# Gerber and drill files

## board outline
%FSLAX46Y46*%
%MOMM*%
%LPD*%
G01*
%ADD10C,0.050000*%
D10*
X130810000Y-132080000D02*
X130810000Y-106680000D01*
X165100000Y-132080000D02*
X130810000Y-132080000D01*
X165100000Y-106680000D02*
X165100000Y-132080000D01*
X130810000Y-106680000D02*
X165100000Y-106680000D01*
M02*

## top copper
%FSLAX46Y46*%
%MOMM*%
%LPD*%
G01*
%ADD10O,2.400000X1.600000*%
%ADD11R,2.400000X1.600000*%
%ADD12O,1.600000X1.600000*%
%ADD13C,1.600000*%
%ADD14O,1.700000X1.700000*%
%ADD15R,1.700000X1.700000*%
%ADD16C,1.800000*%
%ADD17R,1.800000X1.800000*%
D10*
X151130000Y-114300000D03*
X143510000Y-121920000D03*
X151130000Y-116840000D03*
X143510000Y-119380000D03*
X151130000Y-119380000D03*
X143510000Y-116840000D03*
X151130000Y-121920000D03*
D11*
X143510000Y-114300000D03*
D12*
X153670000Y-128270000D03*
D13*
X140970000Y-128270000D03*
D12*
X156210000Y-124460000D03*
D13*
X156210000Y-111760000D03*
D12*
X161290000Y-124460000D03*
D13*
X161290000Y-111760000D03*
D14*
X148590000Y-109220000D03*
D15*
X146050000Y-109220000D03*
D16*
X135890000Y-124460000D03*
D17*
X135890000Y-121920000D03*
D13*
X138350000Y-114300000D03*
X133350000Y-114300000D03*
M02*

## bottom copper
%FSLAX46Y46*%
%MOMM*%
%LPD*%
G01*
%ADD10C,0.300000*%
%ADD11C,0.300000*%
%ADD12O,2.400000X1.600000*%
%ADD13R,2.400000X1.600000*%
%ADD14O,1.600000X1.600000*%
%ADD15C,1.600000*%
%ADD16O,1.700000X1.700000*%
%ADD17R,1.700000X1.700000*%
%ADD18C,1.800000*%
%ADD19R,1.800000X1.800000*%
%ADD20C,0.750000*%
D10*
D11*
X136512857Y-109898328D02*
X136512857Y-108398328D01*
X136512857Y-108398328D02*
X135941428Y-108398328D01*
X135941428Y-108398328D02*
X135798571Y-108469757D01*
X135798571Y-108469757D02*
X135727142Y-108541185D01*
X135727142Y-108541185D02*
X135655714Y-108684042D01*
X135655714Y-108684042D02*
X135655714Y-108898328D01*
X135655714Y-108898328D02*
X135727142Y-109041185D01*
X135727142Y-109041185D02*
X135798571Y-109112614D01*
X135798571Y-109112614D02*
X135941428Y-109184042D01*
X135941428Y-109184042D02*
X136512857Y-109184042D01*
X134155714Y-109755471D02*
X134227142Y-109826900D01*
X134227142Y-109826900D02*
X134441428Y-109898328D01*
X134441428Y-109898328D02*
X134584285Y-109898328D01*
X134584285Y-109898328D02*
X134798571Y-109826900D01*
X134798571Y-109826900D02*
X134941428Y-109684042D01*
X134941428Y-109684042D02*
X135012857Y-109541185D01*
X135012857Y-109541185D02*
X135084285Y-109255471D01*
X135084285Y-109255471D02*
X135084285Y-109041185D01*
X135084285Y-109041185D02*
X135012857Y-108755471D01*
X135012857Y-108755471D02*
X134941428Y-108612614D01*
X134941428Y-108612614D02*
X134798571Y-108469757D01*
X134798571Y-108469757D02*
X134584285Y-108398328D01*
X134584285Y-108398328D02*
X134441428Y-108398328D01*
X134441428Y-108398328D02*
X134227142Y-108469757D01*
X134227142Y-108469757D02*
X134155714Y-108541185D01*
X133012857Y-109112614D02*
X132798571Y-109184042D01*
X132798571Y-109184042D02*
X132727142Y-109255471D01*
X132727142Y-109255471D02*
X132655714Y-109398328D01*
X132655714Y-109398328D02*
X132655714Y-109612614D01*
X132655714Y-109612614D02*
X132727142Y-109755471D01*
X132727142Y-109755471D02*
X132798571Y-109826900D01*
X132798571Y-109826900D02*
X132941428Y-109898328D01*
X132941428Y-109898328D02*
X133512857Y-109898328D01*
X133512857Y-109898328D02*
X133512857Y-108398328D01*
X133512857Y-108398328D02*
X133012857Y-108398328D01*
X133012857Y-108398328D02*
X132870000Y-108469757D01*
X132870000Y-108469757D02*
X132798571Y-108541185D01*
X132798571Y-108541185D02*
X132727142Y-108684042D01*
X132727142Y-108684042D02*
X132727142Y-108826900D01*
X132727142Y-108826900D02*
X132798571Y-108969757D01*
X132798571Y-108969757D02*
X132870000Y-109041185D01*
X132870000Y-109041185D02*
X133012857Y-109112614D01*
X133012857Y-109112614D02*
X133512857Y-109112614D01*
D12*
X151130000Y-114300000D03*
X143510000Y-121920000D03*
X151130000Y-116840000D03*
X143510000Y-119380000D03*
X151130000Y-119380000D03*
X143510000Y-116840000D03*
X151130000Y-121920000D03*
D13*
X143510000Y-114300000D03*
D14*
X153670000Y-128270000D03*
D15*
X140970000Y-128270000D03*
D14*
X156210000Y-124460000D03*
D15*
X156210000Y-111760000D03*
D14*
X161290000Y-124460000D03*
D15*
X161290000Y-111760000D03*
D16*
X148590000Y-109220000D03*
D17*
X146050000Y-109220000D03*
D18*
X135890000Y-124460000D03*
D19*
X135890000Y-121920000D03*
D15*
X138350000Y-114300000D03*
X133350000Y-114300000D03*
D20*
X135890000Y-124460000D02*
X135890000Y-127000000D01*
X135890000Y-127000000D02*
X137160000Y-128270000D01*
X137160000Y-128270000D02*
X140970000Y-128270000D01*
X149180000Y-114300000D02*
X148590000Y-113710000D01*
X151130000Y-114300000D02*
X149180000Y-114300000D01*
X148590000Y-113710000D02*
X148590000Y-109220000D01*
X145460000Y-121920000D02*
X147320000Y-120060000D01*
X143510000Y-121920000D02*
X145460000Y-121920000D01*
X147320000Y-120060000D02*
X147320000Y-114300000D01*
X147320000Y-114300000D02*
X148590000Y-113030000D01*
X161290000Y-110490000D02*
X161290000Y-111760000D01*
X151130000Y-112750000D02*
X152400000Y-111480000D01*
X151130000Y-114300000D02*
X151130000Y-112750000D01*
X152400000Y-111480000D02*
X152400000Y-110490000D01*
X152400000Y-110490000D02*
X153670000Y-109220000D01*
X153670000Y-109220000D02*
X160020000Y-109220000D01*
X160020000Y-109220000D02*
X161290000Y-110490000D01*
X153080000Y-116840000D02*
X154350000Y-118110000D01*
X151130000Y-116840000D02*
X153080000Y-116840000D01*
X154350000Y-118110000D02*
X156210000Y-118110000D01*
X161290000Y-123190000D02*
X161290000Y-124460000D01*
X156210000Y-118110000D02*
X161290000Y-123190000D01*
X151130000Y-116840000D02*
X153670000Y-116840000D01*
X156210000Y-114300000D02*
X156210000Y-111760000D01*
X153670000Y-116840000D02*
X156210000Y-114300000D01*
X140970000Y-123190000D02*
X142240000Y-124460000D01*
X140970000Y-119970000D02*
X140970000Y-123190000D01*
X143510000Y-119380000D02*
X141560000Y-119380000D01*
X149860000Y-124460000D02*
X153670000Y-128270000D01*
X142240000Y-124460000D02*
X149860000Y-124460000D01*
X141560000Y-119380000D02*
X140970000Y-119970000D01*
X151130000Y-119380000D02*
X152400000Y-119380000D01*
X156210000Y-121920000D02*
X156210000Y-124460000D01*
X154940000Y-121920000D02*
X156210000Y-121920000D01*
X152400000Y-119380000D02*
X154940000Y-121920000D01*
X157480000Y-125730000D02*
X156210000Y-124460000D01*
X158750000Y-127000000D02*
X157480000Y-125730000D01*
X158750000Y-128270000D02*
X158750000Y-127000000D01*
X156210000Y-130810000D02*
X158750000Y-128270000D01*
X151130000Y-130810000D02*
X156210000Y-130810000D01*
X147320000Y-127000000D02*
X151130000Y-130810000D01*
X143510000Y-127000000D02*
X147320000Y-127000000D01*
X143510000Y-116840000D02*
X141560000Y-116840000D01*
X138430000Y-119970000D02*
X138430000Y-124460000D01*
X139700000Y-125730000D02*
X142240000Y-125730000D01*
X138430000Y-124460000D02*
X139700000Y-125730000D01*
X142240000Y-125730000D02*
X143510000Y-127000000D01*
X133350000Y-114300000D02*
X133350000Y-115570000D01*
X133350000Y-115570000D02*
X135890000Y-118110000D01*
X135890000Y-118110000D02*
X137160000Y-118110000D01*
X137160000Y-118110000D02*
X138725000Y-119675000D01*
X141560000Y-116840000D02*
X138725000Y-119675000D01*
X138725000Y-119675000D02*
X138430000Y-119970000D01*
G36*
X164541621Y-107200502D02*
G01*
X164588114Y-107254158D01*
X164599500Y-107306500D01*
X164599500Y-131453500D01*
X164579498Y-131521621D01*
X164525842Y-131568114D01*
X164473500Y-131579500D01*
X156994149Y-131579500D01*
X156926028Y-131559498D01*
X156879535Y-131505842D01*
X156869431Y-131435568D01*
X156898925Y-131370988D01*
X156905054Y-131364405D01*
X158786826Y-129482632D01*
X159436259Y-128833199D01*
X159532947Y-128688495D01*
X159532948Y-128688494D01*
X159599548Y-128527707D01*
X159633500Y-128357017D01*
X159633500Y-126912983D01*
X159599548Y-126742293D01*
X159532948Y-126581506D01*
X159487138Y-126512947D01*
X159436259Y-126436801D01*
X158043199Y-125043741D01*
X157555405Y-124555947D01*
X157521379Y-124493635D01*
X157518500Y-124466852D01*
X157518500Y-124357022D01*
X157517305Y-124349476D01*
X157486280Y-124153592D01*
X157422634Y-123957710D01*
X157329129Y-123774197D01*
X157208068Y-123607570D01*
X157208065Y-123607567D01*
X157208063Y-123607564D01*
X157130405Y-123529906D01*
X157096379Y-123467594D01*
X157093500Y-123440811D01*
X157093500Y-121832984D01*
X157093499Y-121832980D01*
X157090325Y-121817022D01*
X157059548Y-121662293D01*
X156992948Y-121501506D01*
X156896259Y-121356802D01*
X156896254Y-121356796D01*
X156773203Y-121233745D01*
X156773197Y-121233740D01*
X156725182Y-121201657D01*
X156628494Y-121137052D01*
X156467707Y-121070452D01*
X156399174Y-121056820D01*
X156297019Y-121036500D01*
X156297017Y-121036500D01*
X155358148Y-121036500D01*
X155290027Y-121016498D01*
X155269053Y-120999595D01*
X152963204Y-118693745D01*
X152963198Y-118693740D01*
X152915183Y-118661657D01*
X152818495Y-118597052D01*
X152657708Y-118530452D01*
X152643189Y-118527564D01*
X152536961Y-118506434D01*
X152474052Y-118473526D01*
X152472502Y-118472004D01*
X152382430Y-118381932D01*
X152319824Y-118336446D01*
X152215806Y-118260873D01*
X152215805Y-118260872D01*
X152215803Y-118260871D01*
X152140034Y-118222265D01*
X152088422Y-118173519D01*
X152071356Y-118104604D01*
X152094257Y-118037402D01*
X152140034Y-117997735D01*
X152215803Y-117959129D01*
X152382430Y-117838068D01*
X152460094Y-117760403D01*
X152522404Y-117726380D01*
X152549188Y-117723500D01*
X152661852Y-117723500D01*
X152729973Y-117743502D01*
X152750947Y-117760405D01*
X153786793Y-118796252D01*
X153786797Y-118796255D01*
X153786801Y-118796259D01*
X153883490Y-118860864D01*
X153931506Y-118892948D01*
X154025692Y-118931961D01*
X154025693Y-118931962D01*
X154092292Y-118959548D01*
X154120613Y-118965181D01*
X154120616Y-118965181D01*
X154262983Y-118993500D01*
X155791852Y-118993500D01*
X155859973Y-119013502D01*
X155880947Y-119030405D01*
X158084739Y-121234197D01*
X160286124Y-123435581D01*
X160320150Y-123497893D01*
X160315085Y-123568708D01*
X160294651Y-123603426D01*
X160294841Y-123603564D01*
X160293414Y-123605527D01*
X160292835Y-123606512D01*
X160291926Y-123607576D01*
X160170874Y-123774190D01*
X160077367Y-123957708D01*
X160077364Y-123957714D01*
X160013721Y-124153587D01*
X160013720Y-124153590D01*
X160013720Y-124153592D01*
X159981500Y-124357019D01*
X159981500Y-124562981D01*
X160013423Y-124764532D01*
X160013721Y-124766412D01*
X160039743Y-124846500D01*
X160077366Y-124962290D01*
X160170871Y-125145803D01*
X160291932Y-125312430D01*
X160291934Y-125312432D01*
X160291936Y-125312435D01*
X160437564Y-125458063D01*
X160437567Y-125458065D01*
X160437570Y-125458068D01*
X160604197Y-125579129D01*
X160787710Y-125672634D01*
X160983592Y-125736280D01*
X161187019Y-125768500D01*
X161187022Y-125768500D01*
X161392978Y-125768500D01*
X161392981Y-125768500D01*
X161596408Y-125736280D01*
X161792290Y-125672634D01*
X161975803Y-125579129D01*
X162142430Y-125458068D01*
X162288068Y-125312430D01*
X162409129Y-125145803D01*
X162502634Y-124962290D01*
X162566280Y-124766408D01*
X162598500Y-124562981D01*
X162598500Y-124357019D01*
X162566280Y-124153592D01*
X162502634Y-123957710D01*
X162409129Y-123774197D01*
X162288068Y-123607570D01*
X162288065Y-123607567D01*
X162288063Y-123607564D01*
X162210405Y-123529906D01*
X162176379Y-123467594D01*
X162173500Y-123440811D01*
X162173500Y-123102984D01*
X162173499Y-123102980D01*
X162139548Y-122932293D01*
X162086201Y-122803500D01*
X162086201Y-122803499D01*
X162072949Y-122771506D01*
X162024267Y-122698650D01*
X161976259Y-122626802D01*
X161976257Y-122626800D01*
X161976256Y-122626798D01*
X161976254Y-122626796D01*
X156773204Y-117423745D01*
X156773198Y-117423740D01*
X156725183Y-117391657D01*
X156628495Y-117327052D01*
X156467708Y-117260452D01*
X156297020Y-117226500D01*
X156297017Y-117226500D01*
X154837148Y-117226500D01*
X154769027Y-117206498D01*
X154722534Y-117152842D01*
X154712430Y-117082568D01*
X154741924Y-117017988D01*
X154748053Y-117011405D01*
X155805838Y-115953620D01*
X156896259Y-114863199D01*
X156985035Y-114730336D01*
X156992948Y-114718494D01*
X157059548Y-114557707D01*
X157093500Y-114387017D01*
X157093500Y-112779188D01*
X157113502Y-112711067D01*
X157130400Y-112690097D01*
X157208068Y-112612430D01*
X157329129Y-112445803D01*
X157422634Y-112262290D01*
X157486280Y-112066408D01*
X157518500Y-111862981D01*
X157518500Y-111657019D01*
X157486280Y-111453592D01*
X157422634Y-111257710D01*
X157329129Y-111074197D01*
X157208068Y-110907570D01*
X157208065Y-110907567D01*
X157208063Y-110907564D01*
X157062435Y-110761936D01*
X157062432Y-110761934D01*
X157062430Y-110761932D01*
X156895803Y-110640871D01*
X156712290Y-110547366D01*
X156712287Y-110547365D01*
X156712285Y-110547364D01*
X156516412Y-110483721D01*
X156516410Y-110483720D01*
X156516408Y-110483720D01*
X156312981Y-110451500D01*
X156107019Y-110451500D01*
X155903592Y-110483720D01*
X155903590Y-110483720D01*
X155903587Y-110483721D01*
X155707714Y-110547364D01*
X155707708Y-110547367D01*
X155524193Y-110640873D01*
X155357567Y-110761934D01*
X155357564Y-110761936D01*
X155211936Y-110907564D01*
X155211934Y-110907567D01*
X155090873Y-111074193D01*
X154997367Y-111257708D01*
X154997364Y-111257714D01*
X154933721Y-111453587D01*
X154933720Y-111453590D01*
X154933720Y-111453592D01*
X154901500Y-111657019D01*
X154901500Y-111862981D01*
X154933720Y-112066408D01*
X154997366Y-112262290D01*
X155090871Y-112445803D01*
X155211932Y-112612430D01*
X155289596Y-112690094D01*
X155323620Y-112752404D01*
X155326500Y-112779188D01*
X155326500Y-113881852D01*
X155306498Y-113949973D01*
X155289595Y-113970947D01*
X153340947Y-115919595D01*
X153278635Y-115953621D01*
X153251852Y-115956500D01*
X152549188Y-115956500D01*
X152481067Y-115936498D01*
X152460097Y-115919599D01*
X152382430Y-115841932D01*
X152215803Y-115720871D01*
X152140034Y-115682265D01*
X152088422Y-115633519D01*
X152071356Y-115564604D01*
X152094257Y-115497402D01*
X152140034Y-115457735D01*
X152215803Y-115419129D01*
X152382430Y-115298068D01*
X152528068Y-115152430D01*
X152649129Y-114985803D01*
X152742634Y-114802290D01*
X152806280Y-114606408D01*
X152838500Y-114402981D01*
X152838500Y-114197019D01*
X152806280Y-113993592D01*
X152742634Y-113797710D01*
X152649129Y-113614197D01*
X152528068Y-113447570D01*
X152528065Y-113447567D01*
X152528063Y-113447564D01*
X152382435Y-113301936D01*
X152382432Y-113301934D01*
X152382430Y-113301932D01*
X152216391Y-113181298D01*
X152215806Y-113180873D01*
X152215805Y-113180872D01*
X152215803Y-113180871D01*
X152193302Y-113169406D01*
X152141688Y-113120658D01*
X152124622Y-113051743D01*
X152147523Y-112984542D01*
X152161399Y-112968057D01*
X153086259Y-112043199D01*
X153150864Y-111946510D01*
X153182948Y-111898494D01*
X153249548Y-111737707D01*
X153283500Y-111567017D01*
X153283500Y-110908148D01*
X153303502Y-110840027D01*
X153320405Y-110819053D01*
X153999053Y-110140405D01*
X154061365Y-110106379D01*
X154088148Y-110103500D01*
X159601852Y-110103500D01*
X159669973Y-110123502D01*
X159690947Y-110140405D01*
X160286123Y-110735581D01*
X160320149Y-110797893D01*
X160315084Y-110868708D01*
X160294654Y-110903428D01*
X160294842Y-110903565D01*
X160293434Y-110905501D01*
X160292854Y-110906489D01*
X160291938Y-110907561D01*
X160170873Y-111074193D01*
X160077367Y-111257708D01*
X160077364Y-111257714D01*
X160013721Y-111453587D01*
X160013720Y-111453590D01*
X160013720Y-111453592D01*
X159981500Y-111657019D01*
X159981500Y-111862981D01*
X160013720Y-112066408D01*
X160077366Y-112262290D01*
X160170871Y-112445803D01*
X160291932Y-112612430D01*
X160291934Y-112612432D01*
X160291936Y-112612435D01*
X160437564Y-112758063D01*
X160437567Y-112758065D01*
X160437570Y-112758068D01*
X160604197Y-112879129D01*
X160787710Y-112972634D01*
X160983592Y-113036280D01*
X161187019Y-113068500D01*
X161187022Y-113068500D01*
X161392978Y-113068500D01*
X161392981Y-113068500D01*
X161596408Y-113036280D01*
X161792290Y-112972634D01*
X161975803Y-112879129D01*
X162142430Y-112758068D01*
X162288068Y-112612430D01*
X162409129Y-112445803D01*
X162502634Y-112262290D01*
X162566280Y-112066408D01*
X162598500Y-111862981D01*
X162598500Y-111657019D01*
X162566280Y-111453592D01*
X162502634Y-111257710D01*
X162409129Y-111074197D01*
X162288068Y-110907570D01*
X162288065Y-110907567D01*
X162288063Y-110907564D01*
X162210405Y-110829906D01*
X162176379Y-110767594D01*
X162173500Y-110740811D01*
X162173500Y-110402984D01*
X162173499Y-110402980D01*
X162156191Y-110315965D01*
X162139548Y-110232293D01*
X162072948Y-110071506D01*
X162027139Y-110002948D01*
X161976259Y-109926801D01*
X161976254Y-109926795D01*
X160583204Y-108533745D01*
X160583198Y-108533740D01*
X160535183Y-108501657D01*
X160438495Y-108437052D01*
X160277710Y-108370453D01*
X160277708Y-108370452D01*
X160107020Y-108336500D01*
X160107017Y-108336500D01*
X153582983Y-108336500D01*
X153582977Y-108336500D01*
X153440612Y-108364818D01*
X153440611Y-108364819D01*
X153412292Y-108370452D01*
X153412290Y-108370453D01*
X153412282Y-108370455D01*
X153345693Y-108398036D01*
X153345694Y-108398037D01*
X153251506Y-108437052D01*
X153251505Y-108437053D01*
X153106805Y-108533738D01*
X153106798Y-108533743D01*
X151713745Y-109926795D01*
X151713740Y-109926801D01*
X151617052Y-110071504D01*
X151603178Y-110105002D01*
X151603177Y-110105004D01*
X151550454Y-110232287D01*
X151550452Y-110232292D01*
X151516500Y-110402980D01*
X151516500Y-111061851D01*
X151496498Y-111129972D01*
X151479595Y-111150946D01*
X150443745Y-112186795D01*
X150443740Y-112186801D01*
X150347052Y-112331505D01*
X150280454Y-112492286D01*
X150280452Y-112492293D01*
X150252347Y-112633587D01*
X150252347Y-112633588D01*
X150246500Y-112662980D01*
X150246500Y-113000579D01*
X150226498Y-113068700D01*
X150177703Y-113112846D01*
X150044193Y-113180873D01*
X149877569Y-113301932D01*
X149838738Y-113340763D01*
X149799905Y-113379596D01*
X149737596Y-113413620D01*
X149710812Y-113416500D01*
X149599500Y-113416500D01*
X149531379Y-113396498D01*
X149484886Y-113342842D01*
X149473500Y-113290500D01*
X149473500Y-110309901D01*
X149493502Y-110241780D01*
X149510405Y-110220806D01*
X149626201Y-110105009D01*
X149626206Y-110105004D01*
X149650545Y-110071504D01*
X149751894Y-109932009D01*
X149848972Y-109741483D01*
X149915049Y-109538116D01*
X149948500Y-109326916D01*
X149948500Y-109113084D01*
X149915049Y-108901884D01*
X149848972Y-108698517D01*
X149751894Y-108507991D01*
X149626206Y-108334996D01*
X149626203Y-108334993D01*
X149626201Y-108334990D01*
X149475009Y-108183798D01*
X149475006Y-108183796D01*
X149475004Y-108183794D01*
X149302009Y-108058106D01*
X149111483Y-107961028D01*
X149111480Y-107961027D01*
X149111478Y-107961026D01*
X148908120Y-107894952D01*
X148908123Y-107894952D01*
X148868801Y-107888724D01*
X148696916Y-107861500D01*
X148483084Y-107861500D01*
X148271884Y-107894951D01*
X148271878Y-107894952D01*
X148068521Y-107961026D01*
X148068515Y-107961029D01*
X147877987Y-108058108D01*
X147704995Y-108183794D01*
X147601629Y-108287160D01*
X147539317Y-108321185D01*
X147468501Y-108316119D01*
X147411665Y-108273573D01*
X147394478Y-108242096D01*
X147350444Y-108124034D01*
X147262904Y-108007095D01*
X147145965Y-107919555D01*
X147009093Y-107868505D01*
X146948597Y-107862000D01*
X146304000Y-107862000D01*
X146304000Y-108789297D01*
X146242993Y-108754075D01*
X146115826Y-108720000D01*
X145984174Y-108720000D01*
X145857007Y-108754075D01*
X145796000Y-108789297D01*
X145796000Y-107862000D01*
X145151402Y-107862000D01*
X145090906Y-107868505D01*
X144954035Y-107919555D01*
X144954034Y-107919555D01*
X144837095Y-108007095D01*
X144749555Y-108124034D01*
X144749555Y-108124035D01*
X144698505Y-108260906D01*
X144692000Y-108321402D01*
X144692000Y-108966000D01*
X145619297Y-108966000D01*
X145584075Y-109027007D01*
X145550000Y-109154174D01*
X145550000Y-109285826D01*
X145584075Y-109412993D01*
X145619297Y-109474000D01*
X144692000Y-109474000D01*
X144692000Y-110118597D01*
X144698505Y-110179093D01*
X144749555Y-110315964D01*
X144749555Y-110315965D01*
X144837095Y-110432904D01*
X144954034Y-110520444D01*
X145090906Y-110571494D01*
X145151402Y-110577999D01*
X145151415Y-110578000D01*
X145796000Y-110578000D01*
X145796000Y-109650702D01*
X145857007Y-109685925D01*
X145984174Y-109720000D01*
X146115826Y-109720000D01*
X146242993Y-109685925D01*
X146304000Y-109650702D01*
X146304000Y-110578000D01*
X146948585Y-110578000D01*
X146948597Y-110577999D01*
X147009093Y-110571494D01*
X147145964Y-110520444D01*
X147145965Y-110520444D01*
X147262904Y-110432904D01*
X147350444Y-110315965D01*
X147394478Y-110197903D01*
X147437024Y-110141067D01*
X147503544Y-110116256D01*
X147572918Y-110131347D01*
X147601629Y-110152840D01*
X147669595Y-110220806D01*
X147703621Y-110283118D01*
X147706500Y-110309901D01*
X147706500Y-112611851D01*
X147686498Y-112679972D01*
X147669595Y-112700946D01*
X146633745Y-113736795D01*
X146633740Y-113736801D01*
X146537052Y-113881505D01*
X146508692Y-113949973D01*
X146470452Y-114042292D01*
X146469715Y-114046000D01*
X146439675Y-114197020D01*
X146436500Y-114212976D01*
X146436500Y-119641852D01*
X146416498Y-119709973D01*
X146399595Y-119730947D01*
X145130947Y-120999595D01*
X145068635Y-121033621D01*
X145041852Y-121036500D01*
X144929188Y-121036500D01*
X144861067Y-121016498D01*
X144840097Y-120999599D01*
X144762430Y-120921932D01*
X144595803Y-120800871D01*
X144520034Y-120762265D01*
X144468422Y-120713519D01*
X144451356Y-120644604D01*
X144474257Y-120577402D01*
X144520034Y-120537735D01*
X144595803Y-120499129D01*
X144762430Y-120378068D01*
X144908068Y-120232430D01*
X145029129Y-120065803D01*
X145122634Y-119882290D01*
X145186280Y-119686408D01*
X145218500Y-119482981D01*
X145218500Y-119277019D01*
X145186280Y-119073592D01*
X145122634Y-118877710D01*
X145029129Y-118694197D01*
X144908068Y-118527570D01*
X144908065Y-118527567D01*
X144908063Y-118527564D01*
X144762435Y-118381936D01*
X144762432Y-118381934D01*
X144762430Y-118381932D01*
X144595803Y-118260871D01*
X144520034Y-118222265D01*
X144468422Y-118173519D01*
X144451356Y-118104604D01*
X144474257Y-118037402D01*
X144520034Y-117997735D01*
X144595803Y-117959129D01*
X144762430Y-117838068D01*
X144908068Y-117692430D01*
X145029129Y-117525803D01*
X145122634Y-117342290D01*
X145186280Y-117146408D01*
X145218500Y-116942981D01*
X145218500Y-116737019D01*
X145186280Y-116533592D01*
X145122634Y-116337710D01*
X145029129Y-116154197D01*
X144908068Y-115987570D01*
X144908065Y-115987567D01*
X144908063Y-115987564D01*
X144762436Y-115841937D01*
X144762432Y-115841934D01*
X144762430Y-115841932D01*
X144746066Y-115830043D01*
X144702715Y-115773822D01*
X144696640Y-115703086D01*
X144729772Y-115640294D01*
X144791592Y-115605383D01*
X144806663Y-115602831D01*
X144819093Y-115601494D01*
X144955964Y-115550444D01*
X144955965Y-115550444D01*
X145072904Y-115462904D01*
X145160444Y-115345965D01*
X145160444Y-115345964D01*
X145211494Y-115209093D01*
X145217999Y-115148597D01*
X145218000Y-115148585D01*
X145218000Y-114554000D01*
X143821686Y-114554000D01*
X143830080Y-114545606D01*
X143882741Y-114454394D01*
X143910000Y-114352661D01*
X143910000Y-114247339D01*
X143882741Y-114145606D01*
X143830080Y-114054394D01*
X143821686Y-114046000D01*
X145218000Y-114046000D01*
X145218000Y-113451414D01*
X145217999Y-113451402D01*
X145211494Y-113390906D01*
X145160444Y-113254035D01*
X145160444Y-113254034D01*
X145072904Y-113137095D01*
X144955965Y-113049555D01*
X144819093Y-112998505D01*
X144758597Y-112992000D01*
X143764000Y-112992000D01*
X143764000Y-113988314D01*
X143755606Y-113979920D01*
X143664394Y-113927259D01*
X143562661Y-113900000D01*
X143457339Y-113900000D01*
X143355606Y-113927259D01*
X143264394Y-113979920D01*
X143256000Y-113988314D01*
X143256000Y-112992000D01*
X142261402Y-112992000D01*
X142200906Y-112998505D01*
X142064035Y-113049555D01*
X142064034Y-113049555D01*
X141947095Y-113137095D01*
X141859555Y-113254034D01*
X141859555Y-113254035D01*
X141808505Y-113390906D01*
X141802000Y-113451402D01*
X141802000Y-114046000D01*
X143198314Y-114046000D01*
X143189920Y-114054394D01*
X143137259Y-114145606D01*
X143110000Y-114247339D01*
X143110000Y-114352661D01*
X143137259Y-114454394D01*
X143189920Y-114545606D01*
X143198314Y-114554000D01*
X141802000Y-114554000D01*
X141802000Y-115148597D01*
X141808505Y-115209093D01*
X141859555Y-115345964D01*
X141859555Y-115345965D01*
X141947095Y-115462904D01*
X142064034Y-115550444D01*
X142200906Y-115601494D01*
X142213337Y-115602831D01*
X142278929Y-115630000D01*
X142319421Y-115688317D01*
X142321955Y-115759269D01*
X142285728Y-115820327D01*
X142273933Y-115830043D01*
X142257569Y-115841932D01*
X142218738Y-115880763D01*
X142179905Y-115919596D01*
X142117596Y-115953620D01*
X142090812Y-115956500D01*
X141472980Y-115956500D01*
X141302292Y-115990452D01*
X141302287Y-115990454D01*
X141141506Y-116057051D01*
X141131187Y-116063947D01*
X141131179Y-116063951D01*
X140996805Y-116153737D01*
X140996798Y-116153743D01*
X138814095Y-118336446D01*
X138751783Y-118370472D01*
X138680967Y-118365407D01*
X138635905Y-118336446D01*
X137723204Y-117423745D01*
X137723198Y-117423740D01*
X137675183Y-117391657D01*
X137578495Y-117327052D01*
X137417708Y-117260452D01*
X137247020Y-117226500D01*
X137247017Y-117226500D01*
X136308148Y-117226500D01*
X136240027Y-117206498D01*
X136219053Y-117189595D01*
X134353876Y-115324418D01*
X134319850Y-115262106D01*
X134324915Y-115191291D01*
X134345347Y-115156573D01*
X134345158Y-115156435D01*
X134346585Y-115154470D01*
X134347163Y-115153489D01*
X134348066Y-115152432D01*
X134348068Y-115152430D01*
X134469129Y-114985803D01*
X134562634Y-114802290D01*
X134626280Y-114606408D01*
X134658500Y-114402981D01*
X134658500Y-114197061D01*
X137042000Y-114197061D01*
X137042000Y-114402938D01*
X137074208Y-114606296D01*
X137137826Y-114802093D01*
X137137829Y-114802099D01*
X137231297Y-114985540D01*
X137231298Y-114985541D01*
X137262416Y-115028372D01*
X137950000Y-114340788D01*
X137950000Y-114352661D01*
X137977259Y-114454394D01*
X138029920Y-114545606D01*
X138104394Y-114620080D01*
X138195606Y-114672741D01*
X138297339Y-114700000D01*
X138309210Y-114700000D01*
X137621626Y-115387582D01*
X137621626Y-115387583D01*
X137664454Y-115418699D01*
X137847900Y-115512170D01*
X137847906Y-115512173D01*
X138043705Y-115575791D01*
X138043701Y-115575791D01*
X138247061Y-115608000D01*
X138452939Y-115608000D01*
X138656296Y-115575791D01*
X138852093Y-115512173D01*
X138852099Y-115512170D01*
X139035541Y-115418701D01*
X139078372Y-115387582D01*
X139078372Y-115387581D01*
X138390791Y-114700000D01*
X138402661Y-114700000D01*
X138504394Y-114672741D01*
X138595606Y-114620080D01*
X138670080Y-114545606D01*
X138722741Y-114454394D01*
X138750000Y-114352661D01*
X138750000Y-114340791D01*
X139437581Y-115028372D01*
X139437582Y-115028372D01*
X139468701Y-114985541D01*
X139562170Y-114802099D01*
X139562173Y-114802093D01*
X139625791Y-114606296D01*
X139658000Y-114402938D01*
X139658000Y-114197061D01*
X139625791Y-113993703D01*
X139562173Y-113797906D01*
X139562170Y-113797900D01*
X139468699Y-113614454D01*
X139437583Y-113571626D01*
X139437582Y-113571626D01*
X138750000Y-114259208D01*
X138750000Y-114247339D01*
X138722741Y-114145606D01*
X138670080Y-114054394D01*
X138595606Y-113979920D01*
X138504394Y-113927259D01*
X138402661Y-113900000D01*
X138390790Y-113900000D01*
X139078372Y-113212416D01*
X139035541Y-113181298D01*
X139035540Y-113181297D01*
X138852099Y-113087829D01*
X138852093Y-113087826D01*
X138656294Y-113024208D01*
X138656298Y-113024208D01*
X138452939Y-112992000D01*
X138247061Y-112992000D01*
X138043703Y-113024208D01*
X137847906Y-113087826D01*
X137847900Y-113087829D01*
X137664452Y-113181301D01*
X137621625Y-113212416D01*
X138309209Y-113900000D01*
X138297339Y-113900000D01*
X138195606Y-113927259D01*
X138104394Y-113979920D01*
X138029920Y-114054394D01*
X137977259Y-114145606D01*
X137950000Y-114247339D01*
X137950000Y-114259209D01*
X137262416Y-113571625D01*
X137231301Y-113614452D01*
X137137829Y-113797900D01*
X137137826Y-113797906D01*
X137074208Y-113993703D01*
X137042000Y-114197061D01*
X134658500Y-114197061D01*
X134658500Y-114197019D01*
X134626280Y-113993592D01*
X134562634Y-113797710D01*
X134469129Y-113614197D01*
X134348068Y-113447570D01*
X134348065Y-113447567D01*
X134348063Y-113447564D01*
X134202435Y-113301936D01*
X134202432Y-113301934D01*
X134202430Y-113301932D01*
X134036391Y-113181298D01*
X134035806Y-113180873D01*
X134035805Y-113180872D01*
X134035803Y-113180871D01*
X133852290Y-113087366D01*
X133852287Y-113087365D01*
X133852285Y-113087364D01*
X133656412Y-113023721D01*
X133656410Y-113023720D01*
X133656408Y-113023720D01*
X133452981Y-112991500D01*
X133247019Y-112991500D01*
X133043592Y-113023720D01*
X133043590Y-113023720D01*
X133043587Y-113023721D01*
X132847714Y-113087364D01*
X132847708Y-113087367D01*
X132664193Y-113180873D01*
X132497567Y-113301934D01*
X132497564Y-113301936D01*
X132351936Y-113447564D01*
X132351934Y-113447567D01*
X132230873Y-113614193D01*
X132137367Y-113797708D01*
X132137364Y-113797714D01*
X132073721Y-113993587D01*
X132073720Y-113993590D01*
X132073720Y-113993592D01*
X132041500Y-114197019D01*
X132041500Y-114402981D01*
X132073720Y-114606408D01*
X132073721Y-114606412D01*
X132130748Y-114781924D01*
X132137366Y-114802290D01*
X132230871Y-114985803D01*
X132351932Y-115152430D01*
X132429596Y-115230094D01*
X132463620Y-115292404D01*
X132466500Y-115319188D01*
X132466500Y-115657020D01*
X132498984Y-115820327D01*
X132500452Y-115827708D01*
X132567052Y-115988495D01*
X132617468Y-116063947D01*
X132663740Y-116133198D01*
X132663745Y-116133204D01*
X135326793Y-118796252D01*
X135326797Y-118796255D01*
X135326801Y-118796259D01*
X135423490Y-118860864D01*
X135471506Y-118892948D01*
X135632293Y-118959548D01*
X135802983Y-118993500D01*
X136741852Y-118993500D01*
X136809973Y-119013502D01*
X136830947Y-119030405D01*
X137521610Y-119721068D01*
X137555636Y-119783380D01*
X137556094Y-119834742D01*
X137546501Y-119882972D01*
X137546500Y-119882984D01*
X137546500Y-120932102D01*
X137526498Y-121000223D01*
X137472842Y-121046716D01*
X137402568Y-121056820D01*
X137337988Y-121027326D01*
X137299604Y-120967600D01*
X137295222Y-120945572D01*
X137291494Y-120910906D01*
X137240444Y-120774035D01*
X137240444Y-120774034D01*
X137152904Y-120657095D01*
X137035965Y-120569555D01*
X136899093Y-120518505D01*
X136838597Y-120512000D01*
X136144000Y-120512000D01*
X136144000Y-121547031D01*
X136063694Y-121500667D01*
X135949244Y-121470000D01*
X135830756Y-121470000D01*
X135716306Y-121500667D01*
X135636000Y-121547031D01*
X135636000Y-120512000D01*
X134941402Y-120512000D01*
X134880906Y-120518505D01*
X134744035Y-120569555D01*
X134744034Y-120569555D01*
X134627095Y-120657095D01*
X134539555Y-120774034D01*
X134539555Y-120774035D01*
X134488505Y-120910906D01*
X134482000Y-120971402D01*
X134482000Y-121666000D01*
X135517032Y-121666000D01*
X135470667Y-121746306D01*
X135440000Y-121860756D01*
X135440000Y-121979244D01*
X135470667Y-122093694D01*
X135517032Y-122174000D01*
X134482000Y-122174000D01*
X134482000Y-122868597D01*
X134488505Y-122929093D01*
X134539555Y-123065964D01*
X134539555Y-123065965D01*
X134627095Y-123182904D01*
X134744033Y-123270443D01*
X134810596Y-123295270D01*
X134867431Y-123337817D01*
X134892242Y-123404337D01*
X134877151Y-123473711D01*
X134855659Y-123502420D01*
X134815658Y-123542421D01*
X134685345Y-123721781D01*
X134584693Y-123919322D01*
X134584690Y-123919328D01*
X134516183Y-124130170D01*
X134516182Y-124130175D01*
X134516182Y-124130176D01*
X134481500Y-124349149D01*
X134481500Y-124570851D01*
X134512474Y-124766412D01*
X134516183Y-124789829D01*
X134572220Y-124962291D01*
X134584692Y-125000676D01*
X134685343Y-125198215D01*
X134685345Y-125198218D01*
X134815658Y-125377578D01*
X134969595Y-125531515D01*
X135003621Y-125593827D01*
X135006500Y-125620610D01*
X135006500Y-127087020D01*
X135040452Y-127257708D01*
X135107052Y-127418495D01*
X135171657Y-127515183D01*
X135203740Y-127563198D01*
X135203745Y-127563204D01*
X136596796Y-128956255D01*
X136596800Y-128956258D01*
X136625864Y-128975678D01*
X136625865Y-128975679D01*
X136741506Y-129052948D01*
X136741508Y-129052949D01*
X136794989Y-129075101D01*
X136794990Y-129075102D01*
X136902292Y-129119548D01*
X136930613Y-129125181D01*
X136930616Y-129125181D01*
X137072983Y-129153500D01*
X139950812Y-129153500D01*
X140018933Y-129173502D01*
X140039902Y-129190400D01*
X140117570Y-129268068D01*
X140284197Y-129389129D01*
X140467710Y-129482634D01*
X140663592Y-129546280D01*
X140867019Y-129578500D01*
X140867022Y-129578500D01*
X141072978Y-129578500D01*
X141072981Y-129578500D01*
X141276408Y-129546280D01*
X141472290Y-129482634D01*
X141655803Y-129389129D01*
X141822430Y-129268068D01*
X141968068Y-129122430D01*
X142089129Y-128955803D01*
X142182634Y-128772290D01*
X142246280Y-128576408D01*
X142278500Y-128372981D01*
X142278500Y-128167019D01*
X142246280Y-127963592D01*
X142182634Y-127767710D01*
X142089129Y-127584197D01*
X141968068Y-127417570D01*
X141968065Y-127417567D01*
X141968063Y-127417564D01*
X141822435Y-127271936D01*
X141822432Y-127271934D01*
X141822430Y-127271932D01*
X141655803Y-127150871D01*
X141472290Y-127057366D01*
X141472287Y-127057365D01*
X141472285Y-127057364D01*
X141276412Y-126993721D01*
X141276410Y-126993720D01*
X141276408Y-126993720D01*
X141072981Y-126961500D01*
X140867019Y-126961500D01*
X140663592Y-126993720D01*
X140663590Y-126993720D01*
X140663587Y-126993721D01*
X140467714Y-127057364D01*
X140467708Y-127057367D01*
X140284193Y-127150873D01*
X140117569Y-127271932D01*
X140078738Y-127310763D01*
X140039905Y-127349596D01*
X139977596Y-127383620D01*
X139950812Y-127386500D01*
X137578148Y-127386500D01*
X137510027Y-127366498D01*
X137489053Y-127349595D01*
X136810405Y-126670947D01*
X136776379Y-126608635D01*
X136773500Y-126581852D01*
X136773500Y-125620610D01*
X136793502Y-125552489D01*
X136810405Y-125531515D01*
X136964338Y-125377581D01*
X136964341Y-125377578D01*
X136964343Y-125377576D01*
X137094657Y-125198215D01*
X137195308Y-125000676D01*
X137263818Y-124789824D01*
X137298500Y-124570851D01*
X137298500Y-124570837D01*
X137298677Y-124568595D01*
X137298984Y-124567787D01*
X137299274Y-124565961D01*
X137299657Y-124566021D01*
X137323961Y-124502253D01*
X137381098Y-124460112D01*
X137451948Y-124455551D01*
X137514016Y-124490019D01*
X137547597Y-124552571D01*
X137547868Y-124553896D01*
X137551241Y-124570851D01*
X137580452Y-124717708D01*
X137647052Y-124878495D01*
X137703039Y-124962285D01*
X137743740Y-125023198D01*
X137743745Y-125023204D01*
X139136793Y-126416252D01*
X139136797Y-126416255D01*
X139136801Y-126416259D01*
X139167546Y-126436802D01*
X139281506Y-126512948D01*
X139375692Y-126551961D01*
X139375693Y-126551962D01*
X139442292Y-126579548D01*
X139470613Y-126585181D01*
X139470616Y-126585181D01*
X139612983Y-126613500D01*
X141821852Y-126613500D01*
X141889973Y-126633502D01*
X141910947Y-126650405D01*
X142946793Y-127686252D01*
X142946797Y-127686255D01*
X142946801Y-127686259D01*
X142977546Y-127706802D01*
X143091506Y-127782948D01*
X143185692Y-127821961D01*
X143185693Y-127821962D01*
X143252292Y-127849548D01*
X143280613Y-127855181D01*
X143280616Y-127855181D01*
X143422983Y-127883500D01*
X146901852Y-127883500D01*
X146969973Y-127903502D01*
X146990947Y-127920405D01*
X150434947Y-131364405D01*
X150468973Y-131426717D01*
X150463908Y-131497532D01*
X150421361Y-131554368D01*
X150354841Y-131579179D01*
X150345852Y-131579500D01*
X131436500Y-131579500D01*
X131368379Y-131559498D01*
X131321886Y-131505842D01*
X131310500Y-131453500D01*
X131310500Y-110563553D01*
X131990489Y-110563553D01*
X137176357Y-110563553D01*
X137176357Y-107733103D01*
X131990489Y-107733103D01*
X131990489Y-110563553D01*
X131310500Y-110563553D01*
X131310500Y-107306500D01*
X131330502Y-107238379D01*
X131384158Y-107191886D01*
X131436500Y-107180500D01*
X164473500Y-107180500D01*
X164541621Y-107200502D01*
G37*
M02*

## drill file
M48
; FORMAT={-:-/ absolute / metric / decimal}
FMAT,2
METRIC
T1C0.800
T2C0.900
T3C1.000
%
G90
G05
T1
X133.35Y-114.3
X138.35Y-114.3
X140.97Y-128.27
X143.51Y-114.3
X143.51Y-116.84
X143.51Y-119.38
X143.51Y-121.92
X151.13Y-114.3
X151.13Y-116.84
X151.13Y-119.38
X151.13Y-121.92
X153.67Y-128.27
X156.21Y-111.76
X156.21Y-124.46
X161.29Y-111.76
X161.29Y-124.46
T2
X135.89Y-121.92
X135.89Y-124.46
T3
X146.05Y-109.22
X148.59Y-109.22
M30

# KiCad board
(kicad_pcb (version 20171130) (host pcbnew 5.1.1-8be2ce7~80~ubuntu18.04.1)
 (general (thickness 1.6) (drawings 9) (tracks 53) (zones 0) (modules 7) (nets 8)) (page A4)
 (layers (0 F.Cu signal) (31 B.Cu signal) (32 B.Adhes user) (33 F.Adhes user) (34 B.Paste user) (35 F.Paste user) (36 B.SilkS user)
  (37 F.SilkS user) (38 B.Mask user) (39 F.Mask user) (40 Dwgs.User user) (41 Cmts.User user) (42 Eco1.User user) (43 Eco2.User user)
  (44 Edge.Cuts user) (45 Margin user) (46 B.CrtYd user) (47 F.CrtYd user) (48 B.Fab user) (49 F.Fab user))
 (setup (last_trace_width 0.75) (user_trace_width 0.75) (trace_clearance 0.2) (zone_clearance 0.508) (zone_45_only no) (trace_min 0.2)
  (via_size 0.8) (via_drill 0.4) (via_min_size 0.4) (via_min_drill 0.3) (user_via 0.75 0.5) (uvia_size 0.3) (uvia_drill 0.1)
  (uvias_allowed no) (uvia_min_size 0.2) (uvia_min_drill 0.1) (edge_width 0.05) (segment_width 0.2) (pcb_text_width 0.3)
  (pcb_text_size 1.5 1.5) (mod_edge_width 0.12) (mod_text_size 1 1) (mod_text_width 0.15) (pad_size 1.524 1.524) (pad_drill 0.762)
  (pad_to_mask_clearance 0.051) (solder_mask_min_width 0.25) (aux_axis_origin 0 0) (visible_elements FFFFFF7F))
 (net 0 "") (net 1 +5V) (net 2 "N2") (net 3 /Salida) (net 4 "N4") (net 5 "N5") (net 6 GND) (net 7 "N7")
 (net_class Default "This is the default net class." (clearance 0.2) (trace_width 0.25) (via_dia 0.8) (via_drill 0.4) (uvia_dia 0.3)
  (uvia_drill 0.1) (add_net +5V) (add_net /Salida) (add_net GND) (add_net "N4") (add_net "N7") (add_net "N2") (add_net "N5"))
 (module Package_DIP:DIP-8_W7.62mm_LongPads (layer F.Cu) (at 143.51 114.3)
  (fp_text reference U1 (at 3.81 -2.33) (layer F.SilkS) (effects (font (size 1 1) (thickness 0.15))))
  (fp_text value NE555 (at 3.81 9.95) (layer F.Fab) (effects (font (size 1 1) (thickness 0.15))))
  (pad 8 thru_hole oval (at 7.62 0) (size 2.4 1.6) (drill 0.8) (layers *.Cu *.Mask) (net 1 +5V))
  (pad 4 thru_hole oval (at 0 7.62) (size 2.4 1.6) (drill 0.8) (layers *.Cu *.Mask) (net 1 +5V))
  (pad 7 thru_hole oval (at 7.62 2.54) (size 2.4 1.6) (drill 0.8) (layers *.Cu *.Mask) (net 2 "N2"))
  (pad 3 thru_hole oval (at 0 5.08) (size 2.4 1.6) (drill 0.8) (layers *.Cu *.Mask) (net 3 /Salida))
  (pad 6 thru_hole oval (at 7.62 5.08) (size 2.4 1.6) (drill 0.8) (layers *.Cu *.Mask) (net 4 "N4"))
  (pad 2 thru_hole oval (at 0 2.54) (size 2.4 1.6) (drill 0.8) (layers *.Cu *.Mask) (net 4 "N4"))
  (pad 5 thru_hole oval (at 7.62 7.62) (size 2.4 1.6) (drill 0.8) (layers *.Cu *.Mask) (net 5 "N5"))
  (pad 1 thru_hole rect (at 0 0) (size 2.4 1.6) (drill 0.8) (layers *.Cu *.Mask) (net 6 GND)))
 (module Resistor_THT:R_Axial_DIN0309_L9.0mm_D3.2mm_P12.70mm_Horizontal (layer F.Cu) (at 140.97 128.27)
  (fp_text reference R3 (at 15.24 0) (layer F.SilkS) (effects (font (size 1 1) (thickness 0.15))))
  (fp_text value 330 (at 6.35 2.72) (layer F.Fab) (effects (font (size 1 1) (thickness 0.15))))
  (pad 2 thru_hole oval (at 12.7 0) (size 1.6 1.6) (drill 0.8) (layers *.Cu *.Mask) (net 3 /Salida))
  (pad 1 thru_hole circle (at 0 0) (size 1.6 1.6) (drill 0.8) (layers *.Cu *.Mask) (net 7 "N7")))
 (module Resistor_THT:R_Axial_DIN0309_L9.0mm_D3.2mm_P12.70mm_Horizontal (layer F.Cu) (at 156.21 111.76 270)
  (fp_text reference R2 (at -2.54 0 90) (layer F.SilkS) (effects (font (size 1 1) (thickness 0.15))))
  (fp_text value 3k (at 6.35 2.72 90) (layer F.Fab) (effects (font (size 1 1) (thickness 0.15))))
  (pad 2 thru_hole oval (at 12.7 0 270) (size 1.6 1.6) (drill 0.8) (layers *.Cu *.Mask) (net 4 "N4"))
  (pad 1 thru_hole circle (at 0 0 270) (size 1.6 1.6) (drill 0.8) (layers *.Cu *.Mask) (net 2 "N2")))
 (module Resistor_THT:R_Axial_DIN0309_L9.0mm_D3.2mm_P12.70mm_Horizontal (layer F.Cu) (at 161.29 111.76 270)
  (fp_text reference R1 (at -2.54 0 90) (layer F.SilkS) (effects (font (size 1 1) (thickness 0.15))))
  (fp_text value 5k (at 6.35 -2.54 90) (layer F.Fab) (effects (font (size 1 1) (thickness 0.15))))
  (pad 2 thru_hole oval (at 12.7 0 270) (size 1.6 1.6) (drill 0.8) (layers *.Cu *.Mask) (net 2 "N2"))
  (pad 1 thru_hole circle (at 0 0 270) (size 1.6 1.6) (drill 0.8) (layers *.Cu *.Mask) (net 1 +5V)))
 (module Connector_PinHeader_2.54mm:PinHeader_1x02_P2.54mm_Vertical (layer F.Cu) (at 146.05 109.22 90)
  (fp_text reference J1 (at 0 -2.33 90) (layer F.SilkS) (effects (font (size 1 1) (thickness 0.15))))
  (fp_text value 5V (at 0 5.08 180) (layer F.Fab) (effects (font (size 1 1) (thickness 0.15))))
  (pad 2 thru_hole oval (at 0 2.54 90) (size 1.7 1.7) (drill 1) (layers *.Cu *.Mask) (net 1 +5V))
  (pad 1 thru_hole rect (at 0 0 90) (size 1.7 1.7) (drill 1) (layers *.Cu *.Mask) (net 6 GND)))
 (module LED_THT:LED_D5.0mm (layer F.Cu) (at 135.89 121.92 270)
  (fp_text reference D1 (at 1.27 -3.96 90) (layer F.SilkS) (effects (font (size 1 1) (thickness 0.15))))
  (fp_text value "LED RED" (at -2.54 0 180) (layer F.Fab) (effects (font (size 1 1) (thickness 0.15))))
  (pad 2 thru_hole circle (at 2.54 0 270) (size 1.8 1.8) (drill 0.9) (layers *.Cu *.Mask) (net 7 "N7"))
  (pad 1 thru_hole rect (at 0 0 270) (size 1.8 1.8) (drill 0.9) (layers *.Cu *.Mask) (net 6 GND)))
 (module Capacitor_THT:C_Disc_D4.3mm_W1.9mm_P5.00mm (layer F.Cu) (at 133.35 114.3)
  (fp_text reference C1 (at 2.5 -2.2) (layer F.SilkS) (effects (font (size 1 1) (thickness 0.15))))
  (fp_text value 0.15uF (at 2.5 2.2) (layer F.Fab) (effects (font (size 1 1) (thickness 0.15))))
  (pad 2 thru_hole circle (at 5 0) (size 1.6 1.6) (drill 0.8) (layers *.Cu *.Mask) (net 6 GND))
  (pad 1 thru_hole circle (at 0 0) (size 1.6 1.6) (drill 0.8) (layers *.Cu *.Mask) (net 4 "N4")))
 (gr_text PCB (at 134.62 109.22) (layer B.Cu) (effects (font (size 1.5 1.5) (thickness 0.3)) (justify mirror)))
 (gr_line (start 130.81 132.08) (end 130.81 106.68) (layer Edge.Cuts) (width 0.05))
 (gr_line (start 165.1 132.08) (end 130.81 132.08) (layer Edge.Cuts) (width 0.05))
 (gr_line (start 165.1 106.68) (end 165.1 132.08) (layer Edge.Cuts) (width 0.05))
 (gr_line (start 130.81 106.68) (end 165.1 106.68) (layer Edge.Cuts) (width 0.05))
 (segment (start 135.89 124.46) (end 135.89 127) (width 0.75) (layer B.Cu) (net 7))
 (segment (start 135.89 127) (end 137.16 128.27) (width 0.75) (layer B.Cu) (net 7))
 (segment (start 137.16 128.27) (end 140.97 128.27) (width 0.75) (layer B.Cu) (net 7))
 (segment (start 149.18 114.3) (end 148.59 113.71) (width 0.75) (layer B.Cu) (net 1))
 (segment (start 151.13 114.3) (end 149.18 114.3) (width 0.75) (layer B.Cu) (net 1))
 (segment (start 148.59 113.71) (end 148.59 109.22) (width 0.75) (layer B.Cu) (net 1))
 (segment (start 145.46 121.92) (end 147.32 120.06) (width 0.75) (layer B.Cu) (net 1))
 (segment (start 143.51 121.92) (end 145.46 121.92) (width 0.75) (layer B.Cu) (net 1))
 (segment (start 147.32 120.06) (end 147.32 114.3) (width 0.75) (layer B.Cu) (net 1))
 (segment (start 147.32 114.3) (end 148.59 113.03) (width 0.75) (layer B.Cu) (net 1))
 (segment (start 161.29 110.49) (end 161.29 111.76) (width 0.75) (layer B.Cu) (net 1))
 (segment (start 151.13 112.75) (end 152.4 111.48) (width 0.75) (layer B.Cu) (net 1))
 (segment (start 151.13 114.3) (end 151.13 112.75) (width 0.75) (layer B.Cu) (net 1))
 (segment (start 152.4 111.48) (end 152.4 110.49) (width 0.75) (layer B.Cu) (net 1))
 (segment (start 152.4 110.49) (end 153.67 109.22) (width 0.75) (layer B.Cu) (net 1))
 (segment (start 153.67 109.22) (end 160.02 109.22) (width 0.75) (layer B.Cu) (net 1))
 (segment (start 160.02 109.22) (end 161.29 110.49) (width 0.75) (layer B.Cu) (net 1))
 (segment (start 153.08 116.84) (end 154.35 118.11) (width 0.75) (layer B.Cu) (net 2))
 (segment (start 151.13 116.84) (end 153.08 116.84) (width 0.75) (layer B.Cu) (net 2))
 (segment (start 154.35 118.11) (end 156.21 118.11) (width 0.75) (layer B.Cu) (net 2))
 (segment (start 161.29 123.19) (end 161.29 124.46) (width 0.75) (layer B.Cu) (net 2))
 (segment (start 156.21 118.11) (end 161.29 123.19) (width 0.75) (layer B.Cu) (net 2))
 (segment (start 151.13 116.84) (end 153.67 116.84) (width 0.75) (layer B.Cu) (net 2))
 (segment (start 156.21 114.3) (end 156.21 111.76) (width 0.75) (layer B.Cu) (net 2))
 (segment (start 153.67 116.84) (end 156.21 114.3) (width 0.75) (layer B.Cu) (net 2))
 (segment (start 140.97 123.19) (end 142.24 124.46) (width 0.75) (layer B.Cu) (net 3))
 (segment (start 140.97 119.97) (end 140.97 123.19) (width 0.75) (layer B.Cu) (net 3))
 (segment (start 143.51 119.38) (end 141.56 119.38) (width 0.75) (layer B.Cu) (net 3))
 (segment (start 149.86 124.46) (end 153.67 128.27) (width 0.75) (layer B.Cu) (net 3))
 (segment (start 142.24 124.46) (end 149.86 124.46) (width 0.75) (layer B.Cu) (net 3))
 (segment (start 141.56 119.38) (end 140.97 119.97) (width 0.75) (layer B.Cu) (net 3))
 (segment (start 151.13 119.38) (end 152.4 119.38) (width 0.75) (layer B.Cu) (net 4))
 (segment (start 156.21 121.92) (end 156.21 124.46) (width 0.75) (layer B.Cu) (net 4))
 (segment (start 154.94 121.92) (end 156.21 121.92) (width 0.75) (layer B.Cu) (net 4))
 (segment (start 152.4 119.38) (end 154.94 121.92) (width 0.75) (layer B.Cu) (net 4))
 (segment (start 157.48 125.73) (end 156.21 124.46) (width 0.75) (layer B.Cu) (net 4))
 (segment (start 158.75 127) (end 157.48 125.73) (width 0.75) (layer B.Cu) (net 4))
 (segment (start 158.75 128.27) (end 158.75 127) (width 0.75) (layer B.Cu) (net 4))
 (segment (start 156.21 130.81) (end 158.75 128.27) (width 0.75) (layer B.Cu) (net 4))
 (segment (start 151.13 130.81) (end 156.21 130.81) (width 0.75) (layer B.Cu) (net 4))
 (segment (start 147.32 127) (end 151.13 130.81) (width 0.75) (layer B.Cu) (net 4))
 (segment (start 143.51 127) (end 147.32 127) (width 0.75) (layer B.Cu) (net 4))
 (segment (start 143.51 116.84) (end 141.56 116.84) (width 0.75) (layer B.Cu) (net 4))
 (segment (start 138.43 119.97) (end 138.43 124.46) (width 0.75) (layer B.Cu) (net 4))
 (segment (start 139.7 125.73) (end 142.24 125.73) (width 0.75) (layer B.Cu) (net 4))
 (segment (start 138.43 124.46) (end 139.7 125.73) (width 0.75) (layer B.Cu) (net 4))
 (segment (start 142.24 125.73) (end 143.51 127) (width 0.75) (layer B.Cu) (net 4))
 (segment (start 133.35 114.3) (end 133.35 115.57) (width 0.75) (layer B.Cu) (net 4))
 (segment (start 133.35 115.57) (end 135.89 118.11) (width 0.75) (layer B.Cu) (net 4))
 (segment (start 135.89 118.11) (end 137.16 118.11) (width 0.75) (layer B.Cu) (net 4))
 (segment (start 137.16 118.11) (end 138.725 119.675) (width 0.75) (layer B.Cu) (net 4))
 (segment (start 141.56 116.84) (end 138.725 119.675) (width 0.75) (layer B.Cu) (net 4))
 (segment (start 138.725 119.675) (end 138.43 119.97) (width 0.75) (layer B.Cu) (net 4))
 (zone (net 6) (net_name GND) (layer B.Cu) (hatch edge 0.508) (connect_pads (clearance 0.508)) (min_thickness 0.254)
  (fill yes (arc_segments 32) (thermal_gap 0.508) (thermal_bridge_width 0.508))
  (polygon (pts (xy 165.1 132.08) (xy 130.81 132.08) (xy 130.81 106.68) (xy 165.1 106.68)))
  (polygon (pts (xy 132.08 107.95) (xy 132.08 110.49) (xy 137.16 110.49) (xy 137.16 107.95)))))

